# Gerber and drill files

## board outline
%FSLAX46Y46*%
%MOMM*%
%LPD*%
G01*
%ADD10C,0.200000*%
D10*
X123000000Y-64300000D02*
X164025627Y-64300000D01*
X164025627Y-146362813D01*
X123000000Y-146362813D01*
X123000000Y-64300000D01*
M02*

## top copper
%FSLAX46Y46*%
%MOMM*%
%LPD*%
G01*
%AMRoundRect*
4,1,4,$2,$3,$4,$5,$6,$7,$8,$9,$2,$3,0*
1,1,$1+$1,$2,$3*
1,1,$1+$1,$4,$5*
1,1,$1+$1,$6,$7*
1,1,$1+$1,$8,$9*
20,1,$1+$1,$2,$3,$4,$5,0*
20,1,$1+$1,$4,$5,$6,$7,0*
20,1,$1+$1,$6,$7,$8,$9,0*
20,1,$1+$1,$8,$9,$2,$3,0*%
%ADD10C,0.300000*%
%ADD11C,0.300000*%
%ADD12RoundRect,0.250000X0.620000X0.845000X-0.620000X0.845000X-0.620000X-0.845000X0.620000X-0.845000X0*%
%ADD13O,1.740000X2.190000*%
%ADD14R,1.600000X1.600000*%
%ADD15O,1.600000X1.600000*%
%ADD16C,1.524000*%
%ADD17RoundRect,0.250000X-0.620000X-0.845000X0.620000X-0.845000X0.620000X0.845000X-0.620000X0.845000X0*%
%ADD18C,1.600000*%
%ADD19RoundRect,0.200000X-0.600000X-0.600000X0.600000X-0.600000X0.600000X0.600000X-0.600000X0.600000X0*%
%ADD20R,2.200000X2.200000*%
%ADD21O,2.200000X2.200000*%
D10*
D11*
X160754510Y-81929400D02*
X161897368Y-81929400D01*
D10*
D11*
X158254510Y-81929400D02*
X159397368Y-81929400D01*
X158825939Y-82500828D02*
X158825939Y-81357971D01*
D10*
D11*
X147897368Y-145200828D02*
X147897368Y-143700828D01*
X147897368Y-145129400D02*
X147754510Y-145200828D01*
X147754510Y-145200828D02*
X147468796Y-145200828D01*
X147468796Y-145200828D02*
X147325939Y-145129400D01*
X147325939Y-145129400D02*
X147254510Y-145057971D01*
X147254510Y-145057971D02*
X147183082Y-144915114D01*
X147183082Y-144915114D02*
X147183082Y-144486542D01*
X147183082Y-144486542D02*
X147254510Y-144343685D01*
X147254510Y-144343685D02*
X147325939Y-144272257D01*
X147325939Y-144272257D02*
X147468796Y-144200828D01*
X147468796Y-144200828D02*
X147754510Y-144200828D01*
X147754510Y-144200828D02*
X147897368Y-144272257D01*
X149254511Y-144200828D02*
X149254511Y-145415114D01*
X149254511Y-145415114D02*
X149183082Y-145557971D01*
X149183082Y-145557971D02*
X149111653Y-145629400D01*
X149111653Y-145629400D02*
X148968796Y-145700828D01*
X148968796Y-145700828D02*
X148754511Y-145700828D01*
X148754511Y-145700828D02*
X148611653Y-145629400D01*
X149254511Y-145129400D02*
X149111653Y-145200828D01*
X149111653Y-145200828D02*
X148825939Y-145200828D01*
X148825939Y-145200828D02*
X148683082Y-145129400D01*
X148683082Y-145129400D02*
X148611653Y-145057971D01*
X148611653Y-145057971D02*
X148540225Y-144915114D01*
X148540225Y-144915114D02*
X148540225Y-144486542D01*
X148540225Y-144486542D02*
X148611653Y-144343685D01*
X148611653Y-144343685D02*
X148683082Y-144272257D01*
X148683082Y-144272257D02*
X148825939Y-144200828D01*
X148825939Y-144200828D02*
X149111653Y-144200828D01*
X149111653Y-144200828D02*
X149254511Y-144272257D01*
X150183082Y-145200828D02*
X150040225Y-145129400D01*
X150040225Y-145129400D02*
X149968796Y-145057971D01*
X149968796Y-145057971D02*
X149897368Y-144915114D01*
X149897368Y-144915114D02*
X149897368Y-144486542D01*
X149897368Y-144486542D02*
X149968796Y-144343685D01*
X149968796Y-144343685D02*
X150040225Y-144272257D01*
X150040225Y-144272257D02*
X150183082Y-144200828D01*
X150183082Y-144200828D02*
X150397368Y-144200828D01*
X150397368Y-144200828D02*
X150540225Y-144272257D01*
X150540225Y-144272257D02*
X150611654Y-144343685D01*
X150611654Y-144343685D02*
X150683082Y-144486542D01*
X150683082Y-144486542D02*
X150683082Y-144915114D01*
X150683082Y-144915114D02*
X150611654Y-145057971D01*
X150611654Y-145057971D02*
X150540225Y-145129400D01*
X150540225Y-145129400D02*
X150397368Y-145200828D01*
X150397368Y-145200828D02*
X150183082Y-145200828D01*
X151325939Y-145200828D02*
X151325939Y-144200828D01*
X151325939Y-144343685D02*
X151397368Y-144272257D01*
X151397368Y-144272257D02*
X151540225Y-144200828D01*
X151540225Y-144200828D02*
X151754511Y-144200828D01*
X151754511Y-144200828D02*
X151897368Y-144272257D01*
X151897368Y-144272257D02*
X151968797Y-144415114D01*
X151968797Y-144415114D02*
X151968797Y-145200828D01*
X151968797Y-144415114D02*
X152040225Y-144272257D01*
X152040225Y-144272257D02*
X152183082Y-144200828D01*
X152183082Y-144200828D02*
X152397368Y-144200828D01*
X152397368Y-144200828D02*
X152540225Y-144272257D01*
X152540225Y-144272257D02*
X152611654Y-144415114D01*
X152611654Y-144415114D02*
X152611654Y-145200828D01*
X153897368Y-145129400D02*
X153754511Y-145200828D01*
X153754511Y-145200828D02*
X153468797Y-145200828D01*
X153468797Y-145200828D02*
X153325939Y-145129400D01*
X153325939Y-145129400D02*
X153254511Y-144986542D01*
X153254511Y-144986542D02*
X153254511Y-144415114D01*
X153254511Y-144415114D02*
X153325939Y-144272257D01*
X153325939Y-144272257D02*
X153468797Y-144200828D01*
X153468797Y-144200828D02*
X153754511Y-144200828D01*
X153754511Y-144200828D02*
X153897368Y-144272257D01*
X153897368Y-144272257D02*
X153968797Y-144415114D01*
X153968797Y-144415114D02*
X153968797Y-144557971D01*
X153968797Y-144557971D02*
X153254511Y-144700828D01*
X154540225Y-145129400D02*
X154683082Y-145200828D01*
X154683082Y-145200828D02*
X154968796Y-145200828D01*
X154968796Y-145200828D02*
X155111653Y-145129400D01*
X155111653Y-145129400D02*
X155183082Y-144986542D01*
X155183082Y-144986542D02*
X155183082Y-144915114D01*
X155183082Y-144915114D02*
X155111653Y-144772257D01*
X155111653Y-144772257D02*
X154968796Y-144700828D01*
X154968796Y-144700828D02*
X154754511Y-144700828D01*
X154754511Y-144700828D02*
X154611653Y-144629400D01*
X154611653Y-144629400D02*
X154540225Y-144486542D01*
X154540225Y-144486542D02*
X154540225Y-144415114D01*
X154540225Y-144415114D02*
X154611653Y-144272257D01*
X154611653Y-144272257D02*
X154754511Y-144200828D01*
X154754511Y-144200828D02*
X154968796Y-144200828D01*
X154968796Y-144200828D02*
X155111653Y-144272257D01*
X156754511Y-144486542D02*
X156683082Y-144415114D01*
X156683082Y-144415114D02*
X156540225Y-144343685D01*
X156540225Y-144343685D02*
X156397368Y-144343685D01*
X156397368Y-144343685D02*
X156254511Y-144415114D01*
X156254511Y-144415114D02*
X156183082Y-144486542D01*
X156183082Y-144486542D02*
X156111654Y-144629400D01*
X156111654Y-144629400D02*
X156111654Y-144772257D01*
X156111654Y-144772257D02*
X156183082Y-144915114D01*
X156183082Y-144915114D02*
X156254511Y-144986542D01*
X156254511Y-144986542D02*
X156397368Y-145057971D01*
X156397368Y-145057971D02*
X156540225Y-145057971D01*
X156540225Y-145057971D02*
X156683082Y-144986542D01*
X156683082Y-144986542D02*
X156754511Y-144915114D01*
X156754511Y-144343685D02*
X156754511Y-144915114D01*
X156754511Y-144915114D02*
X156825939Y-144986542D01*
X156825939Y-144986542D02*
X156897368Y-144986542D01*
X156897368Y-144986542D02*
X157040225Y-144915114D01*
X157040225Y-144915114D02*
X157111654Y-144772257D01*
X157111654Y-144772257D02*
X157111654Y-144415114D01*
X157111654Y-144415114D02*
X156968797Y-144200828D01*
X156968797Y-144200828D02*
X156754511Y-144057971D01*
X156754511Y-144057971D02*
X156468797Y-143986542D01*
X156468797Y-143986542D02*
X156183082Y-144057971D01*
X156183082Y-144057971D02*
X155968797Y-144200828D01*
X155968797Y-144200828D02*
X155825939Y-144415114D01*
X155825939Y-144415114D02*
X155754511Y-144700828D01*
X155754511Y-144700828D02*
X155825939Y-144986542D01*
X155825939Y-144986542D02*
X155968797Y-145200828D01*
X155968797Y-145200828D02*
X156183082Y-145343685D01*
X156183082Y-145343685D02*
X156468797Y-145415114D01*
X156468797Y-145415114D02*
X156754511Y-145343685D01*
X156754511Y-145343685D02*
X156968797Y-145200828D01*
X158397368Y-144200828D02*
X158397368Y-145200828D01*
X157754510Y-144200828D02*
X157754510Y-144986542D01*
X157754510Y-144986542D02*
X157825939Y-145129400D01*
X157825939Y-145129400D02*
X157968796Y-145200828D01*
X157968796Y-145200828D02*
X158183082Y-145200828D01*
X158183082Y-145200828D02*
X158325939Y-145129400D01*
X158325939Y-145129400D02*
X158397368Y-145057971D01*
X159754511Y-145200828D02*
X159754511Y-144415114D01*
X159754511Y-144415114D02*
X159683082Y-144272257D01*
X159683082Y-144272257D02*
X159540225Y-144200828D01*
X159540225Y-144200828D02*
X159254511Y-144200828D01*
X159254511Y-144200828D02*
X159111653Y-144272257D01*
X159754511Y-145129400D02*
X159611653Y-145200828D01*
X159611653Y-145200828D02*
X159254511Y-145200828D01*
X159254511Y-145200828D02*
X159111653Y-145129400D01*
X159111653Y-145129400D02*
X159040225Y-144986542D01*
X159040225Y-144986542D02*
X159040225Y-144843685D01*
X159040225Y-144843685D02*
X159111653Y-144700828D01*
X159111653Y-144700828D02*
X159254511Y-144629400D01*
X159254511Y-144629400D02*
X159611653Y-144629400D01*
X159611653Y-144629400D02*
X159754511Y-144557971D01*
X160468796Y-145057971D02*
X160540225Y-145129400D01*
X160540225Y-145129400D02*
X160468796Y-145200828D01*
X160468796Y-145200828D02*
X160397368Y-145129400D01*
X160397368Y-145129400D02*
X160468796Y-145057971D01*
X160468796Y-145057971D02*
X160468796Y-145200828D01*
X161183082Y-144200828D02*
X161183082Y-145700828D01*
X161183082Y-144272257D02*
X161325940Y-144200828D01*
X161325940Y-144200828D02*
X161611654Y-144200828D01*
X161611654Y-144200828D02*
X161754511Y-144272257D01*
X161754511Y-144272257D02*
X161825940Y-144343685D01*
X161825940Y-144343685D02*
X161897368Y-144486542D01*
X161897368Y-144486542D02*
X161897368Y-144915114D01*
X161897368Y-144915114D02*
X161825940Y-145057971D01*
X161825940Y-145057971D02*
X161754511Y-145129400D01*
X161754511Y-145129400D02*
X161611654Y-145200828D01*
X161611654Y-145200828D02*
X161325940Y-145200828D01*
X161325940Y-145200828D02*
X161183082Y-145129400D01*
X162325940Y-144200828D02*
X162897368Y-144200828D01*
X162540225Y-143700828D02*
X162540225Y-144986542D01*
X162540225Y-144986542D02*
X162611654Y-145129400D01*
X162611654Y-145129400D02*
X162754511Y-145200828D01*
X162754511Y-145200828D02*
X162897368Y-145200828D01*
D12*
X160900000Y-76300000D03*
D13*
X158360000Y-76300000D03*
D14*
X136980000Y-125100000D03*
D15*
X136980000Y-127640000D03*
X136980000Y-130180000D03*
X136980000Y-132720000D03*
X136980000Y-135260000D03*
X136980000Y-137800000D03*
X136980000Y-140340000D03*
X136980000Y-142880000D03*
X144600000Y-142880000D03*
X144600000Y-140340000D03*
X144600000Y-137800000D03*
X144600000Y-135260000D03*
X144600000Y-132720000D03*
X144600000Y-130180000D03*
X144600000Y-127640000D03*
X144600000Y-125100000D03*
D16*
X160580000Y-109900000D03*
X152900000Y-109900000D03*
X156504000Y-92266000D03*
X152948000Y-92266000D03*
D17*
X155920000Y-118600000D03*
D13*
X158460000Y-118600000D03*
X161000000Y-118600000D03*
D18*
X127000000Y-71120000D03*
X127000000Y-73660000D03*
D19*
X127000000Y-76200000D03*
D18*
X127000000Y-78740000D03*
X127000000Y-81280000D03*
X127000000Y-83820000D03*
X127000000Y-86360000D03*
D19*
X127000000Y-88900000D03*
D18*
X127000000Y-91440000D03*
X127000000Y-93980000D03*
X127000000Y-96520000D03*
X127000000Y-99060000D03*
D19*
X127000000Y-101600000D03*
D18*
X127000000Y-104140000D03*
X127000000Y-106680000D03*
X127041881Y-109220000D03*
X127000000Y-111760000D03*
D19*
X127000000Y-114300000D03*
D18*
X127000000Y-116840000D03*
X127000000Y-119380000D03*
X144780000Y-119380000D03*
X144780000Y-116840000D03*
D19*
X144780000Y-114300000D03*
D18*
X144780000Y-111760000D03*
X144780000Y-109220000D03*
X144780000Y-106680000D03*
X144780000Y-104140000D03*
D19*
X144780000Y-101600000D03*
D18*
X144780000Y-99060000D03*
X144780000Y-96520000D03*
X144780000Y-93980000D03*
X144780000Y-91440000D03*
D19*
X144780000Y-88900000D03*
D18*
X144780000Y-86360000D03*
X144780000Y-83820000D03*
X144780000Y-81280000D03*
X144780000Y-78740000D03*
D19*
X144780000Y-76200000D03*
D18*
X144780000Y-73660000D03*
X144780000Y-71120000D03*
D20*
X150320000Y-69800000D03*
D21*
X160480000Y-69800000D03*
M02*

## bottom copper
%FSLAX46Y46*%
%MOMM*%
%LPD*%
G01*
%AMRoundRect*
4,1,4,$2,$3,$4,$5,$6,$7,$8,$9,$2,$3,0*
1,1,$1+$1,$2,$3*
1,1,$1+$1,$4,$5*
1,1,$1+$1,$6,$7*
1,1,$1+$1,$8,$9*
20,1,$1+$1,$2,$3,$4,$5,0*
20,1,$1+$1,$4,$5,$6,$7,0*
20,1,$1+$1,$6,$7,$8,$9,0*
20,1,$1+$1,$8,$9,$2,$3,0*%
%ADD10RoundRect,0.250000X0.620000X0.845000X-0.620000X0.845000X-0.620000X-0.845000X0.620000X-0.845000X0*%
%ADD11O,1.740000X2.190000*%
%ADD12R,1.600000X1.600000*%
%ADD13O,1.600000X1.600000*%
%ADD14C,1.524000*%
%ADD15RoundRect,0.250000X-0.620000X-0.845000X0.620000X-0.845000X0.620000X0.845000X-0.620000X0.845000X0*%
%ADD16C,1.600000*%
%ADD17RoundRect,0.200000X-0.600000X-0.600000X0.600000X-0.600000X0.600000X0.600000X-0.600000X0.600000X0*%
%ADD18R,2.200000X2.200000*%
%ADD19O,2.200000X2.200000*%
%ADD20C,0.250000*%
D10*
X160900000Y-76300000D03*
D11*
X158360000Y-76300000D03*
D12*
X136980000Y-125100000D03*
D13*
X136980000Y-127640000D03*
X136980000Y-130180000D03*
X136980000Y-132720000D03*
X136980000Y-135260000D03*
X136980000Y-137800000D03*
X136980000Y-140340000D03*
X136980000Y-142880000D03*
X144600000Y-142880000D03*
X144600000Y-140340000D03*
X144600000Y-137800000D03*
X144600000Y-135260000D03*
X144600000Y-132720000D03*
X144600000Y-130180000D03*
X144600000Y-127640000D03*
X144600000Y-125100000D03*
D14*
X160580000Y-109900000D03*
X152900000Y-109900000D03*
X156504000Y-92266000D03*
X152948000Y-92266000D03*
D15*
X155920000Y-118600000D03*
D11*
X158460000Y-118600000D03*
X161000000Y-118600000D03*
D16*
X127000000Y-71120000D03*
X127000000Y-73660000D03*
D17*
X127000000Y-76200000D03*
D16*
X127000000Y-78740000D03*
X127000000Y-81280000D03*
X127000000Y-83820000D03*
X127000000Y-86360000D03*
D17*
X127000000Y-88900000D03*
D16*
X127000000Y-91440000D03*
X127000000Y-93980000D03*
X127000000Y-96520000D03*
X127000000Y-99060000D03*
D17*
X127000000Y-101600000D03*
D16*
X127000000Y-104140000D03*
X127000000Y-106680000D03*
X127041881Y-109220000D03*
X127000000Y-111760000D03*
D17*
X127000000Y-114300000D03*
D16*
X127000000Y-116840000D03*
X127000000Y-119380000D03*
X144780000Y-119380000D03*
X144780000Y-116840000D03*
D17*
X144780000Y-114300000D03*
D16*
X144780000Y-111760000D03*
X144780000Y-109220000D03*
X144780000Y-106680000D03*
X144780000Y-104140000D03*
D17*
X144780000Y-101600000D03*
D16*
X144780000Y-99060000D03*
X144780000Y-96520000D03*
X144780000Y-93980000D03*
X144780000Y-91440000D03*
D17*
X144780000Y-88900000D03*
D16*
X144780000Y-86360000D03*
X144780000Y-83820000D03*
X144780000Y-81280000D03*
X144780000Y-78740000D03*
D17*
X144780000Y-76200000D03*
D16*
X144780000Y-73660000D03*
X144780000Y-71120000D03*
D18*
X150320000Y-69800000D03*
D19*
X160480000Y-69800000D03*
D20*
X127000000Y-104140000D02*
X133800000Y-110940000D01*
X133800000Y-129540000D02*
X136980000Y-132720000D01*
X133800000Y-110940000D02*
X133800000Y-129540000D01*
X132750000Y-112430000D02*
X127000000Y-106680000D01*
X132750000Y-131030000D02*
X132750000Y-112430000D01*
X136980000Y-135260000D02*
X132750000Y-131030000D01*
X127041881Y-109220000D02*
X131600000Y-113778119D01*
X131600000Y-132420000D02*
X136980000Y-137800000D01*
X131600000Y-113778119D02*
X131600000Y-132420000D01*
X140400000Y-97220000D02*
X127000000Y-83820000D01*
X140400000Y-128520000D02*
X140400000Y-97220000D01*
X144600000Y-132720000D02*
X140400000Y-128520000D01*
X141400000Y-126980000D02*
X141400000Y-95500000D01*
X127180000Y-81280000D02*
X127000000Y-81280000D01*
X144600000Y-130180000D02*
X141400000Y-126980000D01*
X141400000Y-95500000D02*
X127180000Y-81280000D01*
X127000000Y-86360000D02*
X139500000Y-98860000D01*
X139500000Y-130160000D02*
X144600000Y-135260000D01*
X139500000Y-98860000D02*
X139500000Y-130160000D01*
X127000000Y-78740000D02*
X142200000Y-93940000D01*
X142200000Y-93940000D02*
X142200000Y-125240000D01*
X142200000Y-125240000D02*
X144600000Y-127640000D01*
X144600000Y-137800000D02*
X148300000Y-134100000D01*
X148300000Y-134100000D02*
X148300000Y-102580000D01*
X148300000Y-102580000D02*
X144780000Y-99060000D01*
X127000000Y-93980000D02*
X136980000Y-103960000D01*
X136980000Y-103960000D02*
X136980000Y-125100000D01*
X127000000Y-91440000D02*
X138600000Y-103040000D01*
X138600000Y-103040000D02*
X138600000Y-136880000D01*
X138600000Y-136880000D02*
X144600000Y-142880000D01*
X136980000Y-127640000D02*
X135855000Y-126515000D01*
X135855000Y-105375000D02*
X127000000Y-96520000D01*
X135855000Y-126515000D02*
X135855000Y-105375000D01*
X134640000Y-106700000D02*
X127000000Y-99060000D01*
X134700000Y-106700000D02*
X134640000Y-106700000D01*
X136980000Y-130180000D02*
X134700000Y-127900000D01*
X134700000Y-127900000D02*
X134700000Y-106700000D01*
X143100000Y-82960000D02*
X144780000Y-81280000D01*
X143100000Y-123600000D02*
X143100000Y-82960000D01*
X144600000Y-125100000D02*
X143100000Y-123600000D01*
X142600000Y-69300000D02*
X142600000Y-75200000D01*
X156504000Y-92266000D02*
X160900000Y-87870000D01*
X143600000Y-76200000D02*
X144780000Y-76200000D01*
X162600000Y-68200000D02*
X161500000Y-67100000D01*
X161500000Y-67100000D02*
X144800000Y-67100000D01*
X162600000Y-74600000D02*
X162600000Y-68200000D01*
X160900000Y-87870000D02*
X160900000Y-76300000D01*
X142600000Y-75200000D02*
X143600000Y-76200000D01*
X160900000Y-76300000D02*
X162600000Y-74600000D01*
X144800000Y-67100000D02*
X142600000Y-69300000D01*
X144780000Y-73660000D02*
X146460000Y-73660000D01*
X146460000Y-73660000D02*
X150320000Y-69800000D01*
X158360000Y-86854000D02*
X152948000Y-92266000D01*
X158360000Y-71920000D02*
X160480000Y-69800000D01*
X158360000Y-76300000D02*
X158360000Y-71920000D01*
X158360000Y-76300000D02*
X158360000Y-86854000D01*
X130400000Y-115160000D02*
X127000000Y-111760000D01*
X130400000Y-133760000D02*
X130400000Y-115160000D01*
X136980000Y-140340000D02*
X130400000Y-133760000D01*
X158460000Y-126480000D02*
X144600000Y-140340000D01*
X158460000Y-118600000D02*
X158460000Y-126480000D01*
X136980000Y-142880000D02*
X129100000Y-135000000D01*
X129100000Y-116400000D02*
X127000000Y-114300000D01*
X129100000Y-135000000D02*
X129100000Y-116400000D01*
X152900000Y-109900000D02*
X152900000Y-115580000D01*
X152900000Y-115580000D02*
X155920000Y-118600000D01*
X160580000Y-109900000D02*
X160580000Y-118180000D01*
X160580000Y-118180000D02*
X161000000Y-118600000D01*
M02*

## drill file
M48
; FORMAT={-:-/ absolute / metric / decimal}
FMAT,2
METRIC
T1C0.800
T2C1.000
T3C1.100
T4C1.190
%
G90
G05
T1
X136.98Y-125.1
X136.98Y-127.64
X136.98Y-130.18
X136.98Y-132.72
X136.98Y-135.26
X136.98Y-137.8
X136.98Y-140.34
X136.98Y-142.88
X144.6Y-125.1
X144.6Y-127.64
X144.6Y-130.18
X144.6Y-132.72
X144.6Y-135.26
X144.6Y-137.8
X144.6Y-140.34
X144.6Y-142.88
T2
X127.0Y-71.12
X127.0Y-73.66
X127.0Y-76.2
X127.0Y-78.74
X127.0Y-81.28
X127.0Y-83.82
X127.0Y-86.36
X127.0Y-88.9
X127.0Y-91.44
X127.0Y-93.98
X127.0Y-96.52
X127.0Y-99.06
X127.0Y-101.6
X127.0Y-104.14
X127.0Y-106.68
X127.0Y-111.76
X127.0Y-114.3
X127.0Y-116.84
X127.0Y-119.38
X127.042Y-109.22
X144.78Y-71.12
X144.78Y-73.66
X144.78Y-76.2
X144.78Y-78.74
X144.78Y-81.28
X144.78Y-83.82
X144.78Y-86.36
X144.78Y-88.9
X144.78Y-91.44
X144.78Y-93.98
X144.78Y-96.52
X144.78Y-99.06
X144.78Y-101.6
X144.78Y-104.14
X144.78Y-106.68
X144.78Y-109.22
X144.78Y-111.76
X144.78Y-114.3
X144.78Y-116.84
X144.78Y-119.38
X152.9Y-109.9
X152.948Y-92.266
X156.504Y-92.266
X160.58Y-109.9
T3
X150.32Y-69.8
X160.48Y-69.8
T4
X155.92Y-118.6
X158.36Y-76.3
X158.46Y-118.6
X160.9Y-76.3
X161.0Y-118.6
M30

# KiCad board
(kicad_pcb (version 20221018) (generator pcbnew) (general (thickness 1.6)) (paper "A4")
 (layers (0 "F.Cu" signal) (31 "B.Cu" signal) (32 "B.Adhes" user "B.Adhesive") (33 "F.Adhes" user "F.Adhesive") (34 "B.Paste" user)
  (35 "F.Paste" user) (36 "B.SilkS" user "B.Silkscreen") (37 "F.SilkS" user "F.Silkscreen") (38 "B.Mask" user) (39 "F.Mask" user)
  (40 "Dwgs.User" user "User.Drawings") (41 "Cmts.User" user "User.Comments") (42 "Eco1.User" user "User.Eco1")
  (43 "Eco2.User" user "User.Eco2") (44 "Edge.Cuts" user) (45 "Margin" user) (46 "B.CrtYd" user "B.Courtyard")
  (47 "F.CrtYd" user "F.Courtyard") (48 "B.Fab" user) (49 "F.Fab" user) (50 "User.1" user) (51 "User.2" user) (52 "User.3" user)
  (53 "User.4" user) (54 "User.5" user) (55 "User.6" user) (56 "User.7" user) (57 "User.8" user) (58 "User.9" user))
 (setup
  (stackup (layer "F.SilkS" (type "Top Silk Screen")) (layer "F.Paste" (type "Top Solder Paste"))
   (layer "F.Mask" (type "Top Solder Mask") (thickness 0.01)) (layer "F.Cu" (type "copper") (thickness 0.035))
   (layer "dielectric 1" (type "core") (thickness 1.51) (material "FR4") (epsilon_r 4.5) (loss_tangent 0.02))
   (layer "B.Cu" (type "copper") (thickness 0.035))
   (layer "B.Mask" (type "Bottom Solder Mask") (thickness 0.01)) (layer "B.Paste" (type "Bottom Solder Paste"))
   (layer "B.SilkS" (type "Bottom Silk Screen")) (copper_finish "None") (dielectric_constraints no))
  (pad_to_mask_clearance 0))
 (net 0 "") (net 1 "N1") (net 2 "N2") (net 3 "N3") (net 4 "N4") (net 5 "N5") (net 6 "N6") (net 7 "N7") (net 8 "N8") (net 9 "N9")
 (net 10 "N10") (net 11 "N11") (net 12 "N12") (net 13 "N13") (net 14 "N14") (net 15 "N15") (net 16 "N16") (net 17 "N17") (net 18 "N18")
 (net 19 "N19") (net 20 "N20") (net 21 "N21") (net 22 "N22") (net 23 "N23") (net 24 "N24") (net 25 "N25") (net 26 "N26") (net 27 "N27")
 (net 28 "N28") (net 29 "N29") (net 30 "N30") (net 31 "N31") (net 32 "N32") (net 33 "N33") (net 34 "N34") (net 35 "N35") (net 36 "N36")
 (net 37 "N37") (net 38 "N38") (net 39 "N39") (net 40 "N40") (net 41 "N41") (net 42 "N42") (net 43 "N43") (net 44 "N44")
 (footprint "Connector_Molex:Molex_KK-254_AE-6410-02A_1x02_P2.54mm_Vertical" (layer "F.Cu") (at 160.9 76.3 180)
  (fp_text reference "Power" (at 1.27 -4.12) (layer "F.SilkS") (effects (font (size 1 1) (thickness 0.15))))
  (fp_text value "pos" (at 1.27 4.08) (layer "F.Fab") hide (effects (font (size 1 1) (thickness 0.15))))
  (pad "1" thru_hole roundrect (at 0 0 180) (size 1.74 2.19) (drill 1.19) (layers "*.Cu" "*.Mask") (roundrect_rratio 0.1436781609)
   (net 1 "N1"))
  (pad "2" thru_hole oval (at 2.54 0 180) (size 1.74 2.19) (drill 1.19) (layers "*.Cu" "*.Mask") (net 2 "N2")))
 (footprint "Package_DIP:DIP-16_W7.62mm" (layer "F.Cu") (at 136.98 125.1)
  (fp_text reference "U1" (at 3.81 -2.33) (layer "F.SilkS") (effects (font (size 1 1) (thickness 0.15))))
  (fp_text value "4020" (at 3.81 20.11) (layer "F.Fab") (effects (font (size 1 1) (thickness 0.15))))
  (pad "1" thru_hole rect (at 0 0) (size 1.6 1.6) (drill 0.8) (layers "*.Cu" "*.Mask") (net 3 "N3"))
  (pad "2" thru_hole oval (at 0 2.54) (size 1.6 1.6) (drill 0.8) (layers "*.Cu" "*.Mask") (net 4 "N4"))
  (pad "3" thru_hole oval (at 0 5.08) (size 1.6 1.6) (drill 0.8) (layers "*.Cu" "*.Mask") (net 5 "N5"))
  (pad "4" thru_hole oval (at 0 7.62) (size 1.6 1.6) (drill 0.8) (layers "*.Cu" "*.Mask") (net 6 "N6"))
  (pad "5" thru_hole oval (at 0 10.16) (size 1.6 1.6) (drill 0.8) (layers "*.Cu" "*.Mask") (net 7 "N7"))
  (pad "6" thru_hole oval (at 0 12.7) (size 1.6 1.6) (drill 0.8) (layers "*.Cu" "*.Mask") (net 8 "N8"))
  (pad "7" thru_hole oval (at 0 15.24) (size 1.6 1.6) (drill 0.8) (layers "*.Cu" "*.Mask") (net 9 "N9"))
  (pad "8" thru_hole oval (at 0 17.78) (size 1.6 1.6) (drill 0.8) (layers "*.Cu" "*.Mask") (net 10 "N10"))
  (pad "9" thru_hole oval (at 7.62 17.78) (size 1.6 1.6) (drill 0.8) (layers "*.Cu" "*.Mask") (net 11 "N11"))
  (pad "10" thru_hole oval (at 7.62 15.24) (size 1.6 1.6) (drill 0.8) (layers "*.Cu" "*.Mask") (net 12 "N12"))
  (pad "11" thru_hole oval (at 7.62 12.7) (size 1.6 1.6) (drill 0.8) (layers "*.Cu" "*.Mask") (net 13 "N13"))
  (pad "12" thru_hole oval (at 7.62 10.16) (size 1.6 1.6) (drill 0.8) (layers "*.Cu" "*.Mask") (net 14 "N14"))
  (pad "13" thru_hole oval (at 7.62 7.62) (size 1.6 1.6) (drill 0.8) (layers "*.Cu" "*.Mask") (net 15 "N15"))
  (pad "14" thru_hole oval (at 7.62 5.08) (size 1.6 1.6) (drill 0.8) (layers "*.Cu" "*.Mask") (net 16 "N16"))
  (pad "15" thru_hole oval (at 7.62 2.54) (size 1.6 1.6) (drill 0.8) (layers "*.Cu" "*.Mask") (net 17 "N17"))
  (pad "16" thru_hole oval (at 7.62 0) (size 1.6 1.6) (drill 0.8) (layers "*.Cu" "*.Mask") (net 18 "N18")))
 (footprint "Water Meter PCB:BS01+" (layer "F.Cu") (at 156.504 92.3676 -90)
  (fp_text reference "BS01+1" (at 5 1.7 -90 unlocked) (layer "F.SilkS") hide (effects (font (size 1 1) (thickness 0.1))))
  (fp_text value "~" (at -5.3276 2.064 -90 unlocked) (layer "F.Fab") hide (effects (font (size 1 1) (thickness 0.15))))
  (pad "1" thru_hole circle (at 17.5324 -4.076 270) (size 1.524 1.524) (drill 1) (layers "*.Cu" "*.Mask") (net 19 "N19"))
  (pad "2" thru_hole circle (at 17.5324 3.604 270) (size 1.524 1.524) (drill 1) (layers "*.Cu" "*.Mask") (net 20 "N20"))
  (pad "3" thru_hole circle (at -0.1016 0 270) (size 1.524 1.524) (drill 1) (layers "*.Cu" "*.Mask") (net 1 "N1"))
  (pad "4" thru_hole circle (at -0.1016 3.556 270) (size 1.524 1.524) (drill 1) (layers "*.Cu" "*.Mask") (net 2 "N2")))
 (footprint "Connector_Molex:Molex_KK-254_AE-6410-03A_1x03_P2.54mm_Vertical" (layer "F.Cu") (at 155.92 118.6)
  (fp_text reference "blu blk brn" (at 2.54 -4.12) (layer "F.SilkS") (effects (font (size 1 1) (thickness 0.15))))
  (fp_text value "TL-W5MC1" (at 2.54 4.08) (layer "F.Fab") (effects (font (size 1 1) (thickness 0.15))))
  (pad "1" thru_hole roundrect (at 0 0) (size 1.74 2.19) (drill 1.19) (layers "*.Cu" "*.Mask") (roundrect_rratio 0.1436781609)
   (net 20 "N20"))
  (pad "2" thru_hole oval (at 2.54 0) (size 1.74 2.19) (drill 1.19) (layers "*.Cu" "*.Mask") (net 12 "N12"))
  (pad "3" thru_hole oval (at 5.08 0) (size 1.74 2.19) (drill 1.19) (layers "*.Cu" "*.Mask") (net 19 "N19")))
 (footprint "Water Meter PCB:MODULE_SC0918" (layer "F.Cu") (at 135.89 95.25)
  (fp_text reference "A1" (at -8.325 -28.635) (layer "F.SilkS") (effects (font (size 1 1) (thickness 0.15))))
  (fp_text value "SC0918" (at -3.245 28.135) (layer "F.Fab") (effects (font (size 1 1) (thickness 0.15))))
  (pad "1" thru_hole circle (at -8.89 -24.13) (size 1.6 1.6) (drill 1) (layers "*.Cu" "*.Mask") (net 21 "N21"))
  (pad "2" thru_hole circle (at -8.89 -21.59) (size 1.6 1.6) (drill 1) (layers "*.Cu" "*.Mask") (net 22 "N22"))
  (pad "3" thru_hole roundrect (at -8.89 -19.05) (size 1.6 1.6) (drill 1) (layers "*.Cu" "*.Mask") (roundrect_rratio 0.125) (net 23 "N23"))
  (pad "4" thru_hole circle (at -8.89 -16.51) (size 1.6 1.6) (drill 1) (layers "*.Cu" "*.Mask") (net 17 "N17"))
  (pad "5" thru_hole circle (at -8.89 -13.97) (size 1.6 1.6) (drill 1) (layers "*.Cu" "*.Mask") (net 16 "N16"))
  (pad "6" thru_hole circle (at -8.89 -11.43) (size 1.6 1.6) (drill 1) (layers "*.Cu" "*.Mask") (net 15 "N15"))
  (pad "7" thru_hole circle (at -8.89 -8.89) (size 1.6 1.6) (drill 1) (layers "*.Cu" "*.Mask") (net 14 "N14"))
  (pad "8" thru_hole roundrect (at -8.89 -6.35) (size 1.6 1.6) (drill 1) (layers "*.Cu" "*.Mask") (roundrect_rratio 0.125) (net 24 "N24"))
  (pad "9" thru_hole circle (at -8.89 -3.81) (size 1.6 1.6) (drill 1) (layers "*.Cu" "*.Mask") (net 11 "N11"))
  (pad "10" thru_hole circle (at -8.89 -1.27) (size 1.6 1.6) (drill 1) (layers "*.Cu" "*.Mask") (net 3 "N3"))
  (pad "11" thru_hole circle (at -8.89 1.27) (size 1.6 1.6) (drill 1) (layers "*.Cu" "*.Mask") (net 4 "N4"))
  (pad "12" thru_hole circle (at -8.89 3.81) (size 1.6 1.6) (drill 1) (layers "*.Cu" "*.Mask") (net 5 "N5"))
  (pad "13" thru_hole roundrect (at -8.89 6.35) (size 1.6 1.6) (drill 1) (layers "*.Cu" "*.Mask") (roundrect_rratio 0.125) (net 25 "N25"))
  (pad "14" thru_hole circle (at -8.89 8.89) (size 1.6 1.6) (drill 1) (layers "*.Cu" "*.Mask") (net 6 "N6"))
  (pad "15" thru_hole circle (at -8.89 11.43) (size 1.6 1.6) (drill 1) (layers "*.Cu" "*.Mask") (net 7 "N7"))
  (pad "16" thru_hole circle (at -8.848119 13.97) (size 1.6 1.6) (drill 1) (layers "*.Cu" "*.Mask") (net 8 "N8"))
  (pad "17" thru_hole circle (at -8.89 16.51) (size 1.6 1.6) (drill 1) (layers "*.Cu" "*.Mask") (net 9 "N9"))
  (pad "18" thru_hole roundrect (at -8.89 19.05) (size 1.6 1.6) (drill 1) (layers "*.Cu" "*.Mask") (roundrect_rratio 0.125) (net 10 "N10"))
  (pad "19" thru_hole circle (at -8.89 21.59) (size 1.6 1.6) (drill 1) (layers "*.Cu" "*.Mask") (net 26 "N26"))
  (pad "20" thru_hole circle (at -8.89 24.13) (size 1.6 1.6) (drill 1) (layers "*.Cu" "*.Mask") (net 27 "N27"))
  (pad "21" thru_hole circle (at 8.89 24.13) (size 1.6 1.6) (drill 1) (layers "*.Cu" "*.Mask") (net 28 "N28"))
  (pad "22" thru_hole circle (at 8.89 21.59) (size 1.6 1.6) (drill 1) (layers "*.Cu" "*.Mask") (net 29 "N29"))
  (pad "23" thru_hole roundrect (at 8.89 19.05) (size 1.6 1.6) (drill 1) (layers "*.Cu" "*.Mask") (roundrect_rratio 0.125) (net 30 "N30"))
  (pad "24" thru_hole circle (at 8.89 16.51) (size 1.6 1.6) (drill 1) (layers "*.Cu" "*.Mask") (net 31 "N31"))
  (pad "25" thru_hole circle (at 8.89 13.97) (size 1.6 1.6) (drill 1) (layers "*.Cu" "*.Mask") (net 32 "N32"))
  (pad "26" thru_hole circle (at 8.89 11.43) (size 1.6 1.6) (drill 1) (layers "*.Cu" "*.Mask") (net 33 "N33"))
  (pad "27" thru_hole circle (at 8.89 8.89) (size 1.6 1.6) (drill 1) (layers "*.Cu" "*.Mask") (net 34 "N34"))
  (pad "28" thru_hole roundrect (at 8.89 6.35) (size 1.6 1.6) (drill 1) (layers "*.Cu" "*.Mask") (roundrect_rratio 0.125) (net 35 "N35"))
  (pad "29" thru_hole circle (at 8.89 3.81) (size 1.6 1.6) (drill 1) (layers "*.Cu" "*.Mask") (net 13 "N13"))
  (pad "30" thru_hole circle (at 8.89 1.27) (size 1.6 1.6) (drill 1) (layers "*.Cu" "*.Mask") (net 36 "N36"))
  (pad "31" thru_hole circle (at 8.89 -1.27) (size 1.6 1.6) (drill 1) (layers "*.Cu" "*.Mask") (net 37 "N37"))
  (pad "32" thru_hole circle (at 8.89 -3.81) (size 1.6 1.6) (drill 1) (layers "*.Cu" "*.Mask") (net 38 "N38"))
  (pad "33" thru_hole roundrect (at 8.89 -6.35) (size 1.6 1.6) (drill 1) (layers "*.Cu" "*.Mask") (roundrect_rratio 0.125) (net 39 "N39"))
  (pad "34" thru_hole circle (at 8.89 -8.89) (size 1.6 1.6) (drill 1) (layers "*.Cu" "*.Mask") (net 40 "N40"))
  (pad "35" thru_hole circle (at 8.89 -11.43) (size 1.6 1.6) (drill 1) (layers "*.Cu" "*.Mask") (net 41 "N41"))
  (pad "36" thru_hole circle (at 8.89 -13.97) (size 1.6 1.6) (drill 1) (layers "*.Cu" "*.Mask") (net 18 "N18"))
  (pad "37" thru_hole circle (at 8.89 -16.51) (size 1.6 1.6) (drill 1) (layers "*.Cu" "*.Mask") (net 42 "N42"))
  (pad "38" thru_hole roundrect (at 8.89 -19.05) (size 1.6 1.6) (drill 1) (layers "*.Cu" "*.Mask") (roundrect_rratio 0.125) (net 1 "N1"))
  (pad "39" thru_hole circle (at 8.89 -21.59) (size 1.6 1.6) (drill 1) (layers "*.Cu" "*.Mask") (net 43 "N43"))
  (pad "40" thru_hole circle (at 8.89 -24.13) (size 1.6 1.6) (drill 1) (layers "*.Cu" "*.Mask") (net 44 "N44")))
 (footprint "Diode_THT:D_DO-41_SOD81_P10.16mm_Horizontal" (layer "F.Cu") (at 150.32 69.8)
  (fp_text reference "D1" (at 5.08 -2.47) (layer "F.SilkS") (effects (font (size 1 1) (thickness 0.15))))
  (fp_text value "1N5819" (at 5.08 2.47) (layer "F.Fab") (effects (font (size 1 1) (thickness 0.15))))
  (pad "1" thru_hole rect (at 0 0) (size 2.2 2.2) (drill 1.1) (layers "*.Cu" "*.Mask") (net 43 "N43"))
  (pad "2" thru_hole oval (at 10.16 0) (size 2.2 2.2) (drill 1.1) (layers "*.Cu" "*.Mask") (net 2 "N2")))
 (gr_rect (start 123 64.3) (end 164.025627 146.362813) (stroke (width 0.2) (type default)) (fill none) (layer "Edge.Cuts"))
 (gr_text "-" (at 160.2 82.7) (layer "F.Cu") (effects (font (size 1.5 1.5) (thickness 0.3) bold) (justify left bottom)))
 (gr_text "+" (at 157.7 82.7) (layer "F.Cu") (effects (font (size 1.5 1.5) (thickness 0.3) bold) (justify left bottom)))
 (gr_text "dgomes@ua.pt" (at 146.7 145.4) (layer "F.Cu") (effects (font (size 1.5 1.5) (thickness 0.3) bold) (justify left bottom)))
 (segment (start 127 104.14) (end 133.8 110.94) (width 0.25) (layer "B.Cu") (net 6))
 (segment (start 133.8 129.54) (end 136.98 132.72) (width 0.25) (layer "B.Cu") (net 6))
 (segment (start 133.8 110.94) (end 133.8 129.54) (width 0.25) (layer "B.Cu") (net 6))
 (segment (start 132.75 112.43) (end 127 106.68) (width 0.25) (layer "B.Cu") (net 7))
 (segment (start 132.75 131.03) (end 132.75 112.43) (width 0.25) (layer "B.Cu") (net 7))
 (segment (start 136.98 135.26) (end 132.75 131.03) (width 0.25) (layer "B.Cu") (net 7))
 (segment (start 127.041881 109.22) (end 131.6 113.778119) (width 0.25) (layer "B.Cu") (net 8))
 (segment (start 131.6 132.42) (end 136.98 137.8) (width 0.25) (layer "B.Cu") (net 8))
 (segment (start 131.6 113.778119) (end 131.6 132.42) (width 0.25) (layer "B.Cu") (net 8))
 (segment (start 140.4 97.22) (end 127 83.82) (width 0.25) (layer "B.Cu") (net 15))
 (segment (start 140.4 128.52) (end 140.4 97.22) (width 0.25) (layer "B.Cu") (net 15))
 (segment (start 144.6 132.72) (end 140.4 128.52) (width 0.25) (layer "B.Cu") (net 15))
 (segment (start 141.4 126.98) (end 141.4 95.5) (width 0.25) (layer "B.Cu") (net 16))
 (segment (start 127.18 81.28) (end 127 81.28) (width 0.25) (layer "B.Cu") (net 16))
 (segment (start 144.6 130.18) (end 141.4 126.98) (width 0.25) (layer "B.Cu") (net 16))
 (segment (start 141.4 95.5) (end 127.18 81.28) (width 0.25) (layer "B.Cu") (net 16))
 (segment (start 127 86.36) (end 139.5 98.86) (width 0.25) (layer "B.Cu") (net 14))
 (segment (start 139.5 130.16) (end 144.6 135.26) (width 0.25) (layer "B.Cu") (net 14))
 (segment (start 139.5 98.86) (end 139.5 130.16) (width 0.25) (layer "B.Cu") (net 14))
 (segment (start 127 78.74) (end 142.2 93.94) (width 0.25) (layer "B.Cu") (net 17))
 (segment (start 142.2 93.94) (end 142.2 125.24) (width 0.25) (layer "B.Cu") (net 17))
 (segment (start 142.2 125.24) (end 144.6 127.64) (width 0.25) (layer "B.Cu") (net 17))
 (segment (start 144.6 137.8) (end 148.3 134.1) (width 0.25) (layer "B.Cu") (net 13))
 (segment (start 148.3 134.1) (end 148.3 102.58) (width 0.25) (layer "B.Cu") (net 13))
 (segment (start 148.3 102.58) (end 144.78 99.06) (width 0.25) (layer "B.Cu") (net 13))
 (segment (start 127 93.98) (end 136.98 103.96) (width 0.25) (layer "B.Cu") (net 3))
 (segment (start 136.98 103.96) (end 136.98 125.1) (width 0.25) (layer "B.Cu") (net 3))
 (segment (start 127 91.44) (end 138.6 103.04) (width 0.25) (layer "B.Cu") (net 11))
 (segment (start 138.6 103.04) (end 138.6 136.88) (width 0.25) (layer "B.Cu") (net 11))
 (segment (start 138.6 136.88) (end 144.6 142.88) (width 0.25) (layer "B.Cu") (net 11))
 (segment (start 136.98 127.64) (end 135.855 126.515) (width 0.25) (layer "B.Cu") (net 4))
 (segment (start 135.855 105.375) (end 127 96.52) (width 0.25) (layer "B.Cu") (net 4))
 (segment (start 135.855 126.515) (end 135.855 105.375) (width 0.25) (layer "B.Cu") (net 4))
 (segment (start 134.64 106.7) (end 127 99.06) (width 0.25) (layer "B.Cu") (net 5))
 (segment (start 134.7 106.7) (end 134.64 106.7) (width 0.25) (layer "B.Cu") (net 5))
 (segment (start 136.98 130.18) (end 134.7 127.9) (width 0.25) (layer "B.Cu") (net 5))
 (segment (start 134.7 127.9) (end 134.7 106.7) (width 0.25) (layer "B.Cu") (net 5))
 (segment (start 143.1 82.96) (end 144.78 81.28) (width 0.25) (layer "B.Cu") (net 18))
 (segment (start 143.1 123.6) (end 143.1 82.96) (width 0.25) (layer "B.Cu") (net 18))
 (segment (start 144.6 125.1) (end 143.1 123.6) (width 0.25) (layer "B.Cu") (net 18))
 (segment (start 142.6 69.3) (end 142.6 75.2) (width 0.25) (layer "B.Cu") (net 1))
 (segment (start 156.504 92.266) (end 160.9 87.87) (width 0.25) (layer "B.Cu") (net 1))
 (segment (start 143.6 76.2) (end 144.78 76.2) (width 0.25) (layer "B.Cu") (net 1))
 (segment (start 162.6 68.2) (end 161.5 67.1) (width 0.25) (layer "B.Cu") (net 1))
 (segment (start 161.5 67.1) (end 144.8 67.1) (width 0.25) (layer "B.Cu") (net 1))
 (segment (start 162.6 74.6) (end 162.6 68.2) (width 0.25) (layer "B.Cu") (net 1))
 (segment (start 160.9 87.87) (end 160.9 76.3) (width 0.25) (layer "B.Cu") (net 1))
 (segment (start 142.6 75.2) (end 143.6 76.2) (width 0.25) (layer "B.Cu") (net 1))
 (segment (start 160.9 76.3) (end 162.6 74.6) (width 0.25) (layer "B.Cu") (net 1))
 (segment (start 144.8 67.1) (end 142.6 69.3) (width 0.25) (layer "B.Cu") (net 1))
 (segment (start 144.78 73.66) (end 146.46 73.66) (width 0.25) (layer "B.Cu") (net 43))
 (segment (start 146.46 73.66) (end 150.32 69.8) (width 0.25) (layer "B.Cu") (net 43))
 (segment (start 158.36 86.854) (end 152.948 92.266) (width 0.25) (layer "B.Cu") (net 2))
 (segment (start 158.36 71.92) (end 160.48 69.8) (width 0.25) (layer "B.Cu") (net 2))
 (segment (start 158.36 76.3) (end 158.36 71.92) (width 0.25) (layer "B.Cu") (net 2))
 (segment (start 158.36 76.3) (end 158.36 86.854) (width 0.25) (layer "B.Cu") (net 2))
 (segment (start 130.4 115.16) (end 127 111.76) (width 0.25) (layer "B.Cu") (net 9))
 (segment (start 130.4 133.76) (end 130.4 115.16) (width 0.25) (layer "B.Cu") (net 9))
 (segment (start 136.98 140.34) (end 130.4 133.76) (width 0.25) (layer "B.Cu") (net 9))
 (segment (start 158.46 126.48) (end 144.6 140.34) (width 0.25) (layer "B.Cu") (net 12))
 (segment (start 158.46 118.6) (end 158.46 126.48) (width 0.25) (layer "B.Cu") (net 12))
 (segment (start 136.98 142.88) (end 129.1 135) (width 0.25) (layer "B.Cu") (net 10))
 (segment (start 129.1 116.4) (end 127 114.3) (width 0.25) (layer "B.Cu") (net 10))
 (segment (start 129.1 135) (end 129.1 116.4) (width 0.25) (layer "B.Cu") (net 10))
 (segment (start 152.9 109.9) (end 152.9 115.58) (width 0.25) (layer "B.Cu") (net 20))
 (segment (start 152.9 115.58) (end 155.92 118.6) (width 0.25) (layer "B.Cu") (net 20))
 (segment (start 160.58 109.9) (end 160.58 118.18) (width 0.25) (layer "B.Cu") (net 19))
 (segment (start 160.58 118.18) (end 161 118.6) (width 0.25) (layer "B.Cu") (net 19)))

